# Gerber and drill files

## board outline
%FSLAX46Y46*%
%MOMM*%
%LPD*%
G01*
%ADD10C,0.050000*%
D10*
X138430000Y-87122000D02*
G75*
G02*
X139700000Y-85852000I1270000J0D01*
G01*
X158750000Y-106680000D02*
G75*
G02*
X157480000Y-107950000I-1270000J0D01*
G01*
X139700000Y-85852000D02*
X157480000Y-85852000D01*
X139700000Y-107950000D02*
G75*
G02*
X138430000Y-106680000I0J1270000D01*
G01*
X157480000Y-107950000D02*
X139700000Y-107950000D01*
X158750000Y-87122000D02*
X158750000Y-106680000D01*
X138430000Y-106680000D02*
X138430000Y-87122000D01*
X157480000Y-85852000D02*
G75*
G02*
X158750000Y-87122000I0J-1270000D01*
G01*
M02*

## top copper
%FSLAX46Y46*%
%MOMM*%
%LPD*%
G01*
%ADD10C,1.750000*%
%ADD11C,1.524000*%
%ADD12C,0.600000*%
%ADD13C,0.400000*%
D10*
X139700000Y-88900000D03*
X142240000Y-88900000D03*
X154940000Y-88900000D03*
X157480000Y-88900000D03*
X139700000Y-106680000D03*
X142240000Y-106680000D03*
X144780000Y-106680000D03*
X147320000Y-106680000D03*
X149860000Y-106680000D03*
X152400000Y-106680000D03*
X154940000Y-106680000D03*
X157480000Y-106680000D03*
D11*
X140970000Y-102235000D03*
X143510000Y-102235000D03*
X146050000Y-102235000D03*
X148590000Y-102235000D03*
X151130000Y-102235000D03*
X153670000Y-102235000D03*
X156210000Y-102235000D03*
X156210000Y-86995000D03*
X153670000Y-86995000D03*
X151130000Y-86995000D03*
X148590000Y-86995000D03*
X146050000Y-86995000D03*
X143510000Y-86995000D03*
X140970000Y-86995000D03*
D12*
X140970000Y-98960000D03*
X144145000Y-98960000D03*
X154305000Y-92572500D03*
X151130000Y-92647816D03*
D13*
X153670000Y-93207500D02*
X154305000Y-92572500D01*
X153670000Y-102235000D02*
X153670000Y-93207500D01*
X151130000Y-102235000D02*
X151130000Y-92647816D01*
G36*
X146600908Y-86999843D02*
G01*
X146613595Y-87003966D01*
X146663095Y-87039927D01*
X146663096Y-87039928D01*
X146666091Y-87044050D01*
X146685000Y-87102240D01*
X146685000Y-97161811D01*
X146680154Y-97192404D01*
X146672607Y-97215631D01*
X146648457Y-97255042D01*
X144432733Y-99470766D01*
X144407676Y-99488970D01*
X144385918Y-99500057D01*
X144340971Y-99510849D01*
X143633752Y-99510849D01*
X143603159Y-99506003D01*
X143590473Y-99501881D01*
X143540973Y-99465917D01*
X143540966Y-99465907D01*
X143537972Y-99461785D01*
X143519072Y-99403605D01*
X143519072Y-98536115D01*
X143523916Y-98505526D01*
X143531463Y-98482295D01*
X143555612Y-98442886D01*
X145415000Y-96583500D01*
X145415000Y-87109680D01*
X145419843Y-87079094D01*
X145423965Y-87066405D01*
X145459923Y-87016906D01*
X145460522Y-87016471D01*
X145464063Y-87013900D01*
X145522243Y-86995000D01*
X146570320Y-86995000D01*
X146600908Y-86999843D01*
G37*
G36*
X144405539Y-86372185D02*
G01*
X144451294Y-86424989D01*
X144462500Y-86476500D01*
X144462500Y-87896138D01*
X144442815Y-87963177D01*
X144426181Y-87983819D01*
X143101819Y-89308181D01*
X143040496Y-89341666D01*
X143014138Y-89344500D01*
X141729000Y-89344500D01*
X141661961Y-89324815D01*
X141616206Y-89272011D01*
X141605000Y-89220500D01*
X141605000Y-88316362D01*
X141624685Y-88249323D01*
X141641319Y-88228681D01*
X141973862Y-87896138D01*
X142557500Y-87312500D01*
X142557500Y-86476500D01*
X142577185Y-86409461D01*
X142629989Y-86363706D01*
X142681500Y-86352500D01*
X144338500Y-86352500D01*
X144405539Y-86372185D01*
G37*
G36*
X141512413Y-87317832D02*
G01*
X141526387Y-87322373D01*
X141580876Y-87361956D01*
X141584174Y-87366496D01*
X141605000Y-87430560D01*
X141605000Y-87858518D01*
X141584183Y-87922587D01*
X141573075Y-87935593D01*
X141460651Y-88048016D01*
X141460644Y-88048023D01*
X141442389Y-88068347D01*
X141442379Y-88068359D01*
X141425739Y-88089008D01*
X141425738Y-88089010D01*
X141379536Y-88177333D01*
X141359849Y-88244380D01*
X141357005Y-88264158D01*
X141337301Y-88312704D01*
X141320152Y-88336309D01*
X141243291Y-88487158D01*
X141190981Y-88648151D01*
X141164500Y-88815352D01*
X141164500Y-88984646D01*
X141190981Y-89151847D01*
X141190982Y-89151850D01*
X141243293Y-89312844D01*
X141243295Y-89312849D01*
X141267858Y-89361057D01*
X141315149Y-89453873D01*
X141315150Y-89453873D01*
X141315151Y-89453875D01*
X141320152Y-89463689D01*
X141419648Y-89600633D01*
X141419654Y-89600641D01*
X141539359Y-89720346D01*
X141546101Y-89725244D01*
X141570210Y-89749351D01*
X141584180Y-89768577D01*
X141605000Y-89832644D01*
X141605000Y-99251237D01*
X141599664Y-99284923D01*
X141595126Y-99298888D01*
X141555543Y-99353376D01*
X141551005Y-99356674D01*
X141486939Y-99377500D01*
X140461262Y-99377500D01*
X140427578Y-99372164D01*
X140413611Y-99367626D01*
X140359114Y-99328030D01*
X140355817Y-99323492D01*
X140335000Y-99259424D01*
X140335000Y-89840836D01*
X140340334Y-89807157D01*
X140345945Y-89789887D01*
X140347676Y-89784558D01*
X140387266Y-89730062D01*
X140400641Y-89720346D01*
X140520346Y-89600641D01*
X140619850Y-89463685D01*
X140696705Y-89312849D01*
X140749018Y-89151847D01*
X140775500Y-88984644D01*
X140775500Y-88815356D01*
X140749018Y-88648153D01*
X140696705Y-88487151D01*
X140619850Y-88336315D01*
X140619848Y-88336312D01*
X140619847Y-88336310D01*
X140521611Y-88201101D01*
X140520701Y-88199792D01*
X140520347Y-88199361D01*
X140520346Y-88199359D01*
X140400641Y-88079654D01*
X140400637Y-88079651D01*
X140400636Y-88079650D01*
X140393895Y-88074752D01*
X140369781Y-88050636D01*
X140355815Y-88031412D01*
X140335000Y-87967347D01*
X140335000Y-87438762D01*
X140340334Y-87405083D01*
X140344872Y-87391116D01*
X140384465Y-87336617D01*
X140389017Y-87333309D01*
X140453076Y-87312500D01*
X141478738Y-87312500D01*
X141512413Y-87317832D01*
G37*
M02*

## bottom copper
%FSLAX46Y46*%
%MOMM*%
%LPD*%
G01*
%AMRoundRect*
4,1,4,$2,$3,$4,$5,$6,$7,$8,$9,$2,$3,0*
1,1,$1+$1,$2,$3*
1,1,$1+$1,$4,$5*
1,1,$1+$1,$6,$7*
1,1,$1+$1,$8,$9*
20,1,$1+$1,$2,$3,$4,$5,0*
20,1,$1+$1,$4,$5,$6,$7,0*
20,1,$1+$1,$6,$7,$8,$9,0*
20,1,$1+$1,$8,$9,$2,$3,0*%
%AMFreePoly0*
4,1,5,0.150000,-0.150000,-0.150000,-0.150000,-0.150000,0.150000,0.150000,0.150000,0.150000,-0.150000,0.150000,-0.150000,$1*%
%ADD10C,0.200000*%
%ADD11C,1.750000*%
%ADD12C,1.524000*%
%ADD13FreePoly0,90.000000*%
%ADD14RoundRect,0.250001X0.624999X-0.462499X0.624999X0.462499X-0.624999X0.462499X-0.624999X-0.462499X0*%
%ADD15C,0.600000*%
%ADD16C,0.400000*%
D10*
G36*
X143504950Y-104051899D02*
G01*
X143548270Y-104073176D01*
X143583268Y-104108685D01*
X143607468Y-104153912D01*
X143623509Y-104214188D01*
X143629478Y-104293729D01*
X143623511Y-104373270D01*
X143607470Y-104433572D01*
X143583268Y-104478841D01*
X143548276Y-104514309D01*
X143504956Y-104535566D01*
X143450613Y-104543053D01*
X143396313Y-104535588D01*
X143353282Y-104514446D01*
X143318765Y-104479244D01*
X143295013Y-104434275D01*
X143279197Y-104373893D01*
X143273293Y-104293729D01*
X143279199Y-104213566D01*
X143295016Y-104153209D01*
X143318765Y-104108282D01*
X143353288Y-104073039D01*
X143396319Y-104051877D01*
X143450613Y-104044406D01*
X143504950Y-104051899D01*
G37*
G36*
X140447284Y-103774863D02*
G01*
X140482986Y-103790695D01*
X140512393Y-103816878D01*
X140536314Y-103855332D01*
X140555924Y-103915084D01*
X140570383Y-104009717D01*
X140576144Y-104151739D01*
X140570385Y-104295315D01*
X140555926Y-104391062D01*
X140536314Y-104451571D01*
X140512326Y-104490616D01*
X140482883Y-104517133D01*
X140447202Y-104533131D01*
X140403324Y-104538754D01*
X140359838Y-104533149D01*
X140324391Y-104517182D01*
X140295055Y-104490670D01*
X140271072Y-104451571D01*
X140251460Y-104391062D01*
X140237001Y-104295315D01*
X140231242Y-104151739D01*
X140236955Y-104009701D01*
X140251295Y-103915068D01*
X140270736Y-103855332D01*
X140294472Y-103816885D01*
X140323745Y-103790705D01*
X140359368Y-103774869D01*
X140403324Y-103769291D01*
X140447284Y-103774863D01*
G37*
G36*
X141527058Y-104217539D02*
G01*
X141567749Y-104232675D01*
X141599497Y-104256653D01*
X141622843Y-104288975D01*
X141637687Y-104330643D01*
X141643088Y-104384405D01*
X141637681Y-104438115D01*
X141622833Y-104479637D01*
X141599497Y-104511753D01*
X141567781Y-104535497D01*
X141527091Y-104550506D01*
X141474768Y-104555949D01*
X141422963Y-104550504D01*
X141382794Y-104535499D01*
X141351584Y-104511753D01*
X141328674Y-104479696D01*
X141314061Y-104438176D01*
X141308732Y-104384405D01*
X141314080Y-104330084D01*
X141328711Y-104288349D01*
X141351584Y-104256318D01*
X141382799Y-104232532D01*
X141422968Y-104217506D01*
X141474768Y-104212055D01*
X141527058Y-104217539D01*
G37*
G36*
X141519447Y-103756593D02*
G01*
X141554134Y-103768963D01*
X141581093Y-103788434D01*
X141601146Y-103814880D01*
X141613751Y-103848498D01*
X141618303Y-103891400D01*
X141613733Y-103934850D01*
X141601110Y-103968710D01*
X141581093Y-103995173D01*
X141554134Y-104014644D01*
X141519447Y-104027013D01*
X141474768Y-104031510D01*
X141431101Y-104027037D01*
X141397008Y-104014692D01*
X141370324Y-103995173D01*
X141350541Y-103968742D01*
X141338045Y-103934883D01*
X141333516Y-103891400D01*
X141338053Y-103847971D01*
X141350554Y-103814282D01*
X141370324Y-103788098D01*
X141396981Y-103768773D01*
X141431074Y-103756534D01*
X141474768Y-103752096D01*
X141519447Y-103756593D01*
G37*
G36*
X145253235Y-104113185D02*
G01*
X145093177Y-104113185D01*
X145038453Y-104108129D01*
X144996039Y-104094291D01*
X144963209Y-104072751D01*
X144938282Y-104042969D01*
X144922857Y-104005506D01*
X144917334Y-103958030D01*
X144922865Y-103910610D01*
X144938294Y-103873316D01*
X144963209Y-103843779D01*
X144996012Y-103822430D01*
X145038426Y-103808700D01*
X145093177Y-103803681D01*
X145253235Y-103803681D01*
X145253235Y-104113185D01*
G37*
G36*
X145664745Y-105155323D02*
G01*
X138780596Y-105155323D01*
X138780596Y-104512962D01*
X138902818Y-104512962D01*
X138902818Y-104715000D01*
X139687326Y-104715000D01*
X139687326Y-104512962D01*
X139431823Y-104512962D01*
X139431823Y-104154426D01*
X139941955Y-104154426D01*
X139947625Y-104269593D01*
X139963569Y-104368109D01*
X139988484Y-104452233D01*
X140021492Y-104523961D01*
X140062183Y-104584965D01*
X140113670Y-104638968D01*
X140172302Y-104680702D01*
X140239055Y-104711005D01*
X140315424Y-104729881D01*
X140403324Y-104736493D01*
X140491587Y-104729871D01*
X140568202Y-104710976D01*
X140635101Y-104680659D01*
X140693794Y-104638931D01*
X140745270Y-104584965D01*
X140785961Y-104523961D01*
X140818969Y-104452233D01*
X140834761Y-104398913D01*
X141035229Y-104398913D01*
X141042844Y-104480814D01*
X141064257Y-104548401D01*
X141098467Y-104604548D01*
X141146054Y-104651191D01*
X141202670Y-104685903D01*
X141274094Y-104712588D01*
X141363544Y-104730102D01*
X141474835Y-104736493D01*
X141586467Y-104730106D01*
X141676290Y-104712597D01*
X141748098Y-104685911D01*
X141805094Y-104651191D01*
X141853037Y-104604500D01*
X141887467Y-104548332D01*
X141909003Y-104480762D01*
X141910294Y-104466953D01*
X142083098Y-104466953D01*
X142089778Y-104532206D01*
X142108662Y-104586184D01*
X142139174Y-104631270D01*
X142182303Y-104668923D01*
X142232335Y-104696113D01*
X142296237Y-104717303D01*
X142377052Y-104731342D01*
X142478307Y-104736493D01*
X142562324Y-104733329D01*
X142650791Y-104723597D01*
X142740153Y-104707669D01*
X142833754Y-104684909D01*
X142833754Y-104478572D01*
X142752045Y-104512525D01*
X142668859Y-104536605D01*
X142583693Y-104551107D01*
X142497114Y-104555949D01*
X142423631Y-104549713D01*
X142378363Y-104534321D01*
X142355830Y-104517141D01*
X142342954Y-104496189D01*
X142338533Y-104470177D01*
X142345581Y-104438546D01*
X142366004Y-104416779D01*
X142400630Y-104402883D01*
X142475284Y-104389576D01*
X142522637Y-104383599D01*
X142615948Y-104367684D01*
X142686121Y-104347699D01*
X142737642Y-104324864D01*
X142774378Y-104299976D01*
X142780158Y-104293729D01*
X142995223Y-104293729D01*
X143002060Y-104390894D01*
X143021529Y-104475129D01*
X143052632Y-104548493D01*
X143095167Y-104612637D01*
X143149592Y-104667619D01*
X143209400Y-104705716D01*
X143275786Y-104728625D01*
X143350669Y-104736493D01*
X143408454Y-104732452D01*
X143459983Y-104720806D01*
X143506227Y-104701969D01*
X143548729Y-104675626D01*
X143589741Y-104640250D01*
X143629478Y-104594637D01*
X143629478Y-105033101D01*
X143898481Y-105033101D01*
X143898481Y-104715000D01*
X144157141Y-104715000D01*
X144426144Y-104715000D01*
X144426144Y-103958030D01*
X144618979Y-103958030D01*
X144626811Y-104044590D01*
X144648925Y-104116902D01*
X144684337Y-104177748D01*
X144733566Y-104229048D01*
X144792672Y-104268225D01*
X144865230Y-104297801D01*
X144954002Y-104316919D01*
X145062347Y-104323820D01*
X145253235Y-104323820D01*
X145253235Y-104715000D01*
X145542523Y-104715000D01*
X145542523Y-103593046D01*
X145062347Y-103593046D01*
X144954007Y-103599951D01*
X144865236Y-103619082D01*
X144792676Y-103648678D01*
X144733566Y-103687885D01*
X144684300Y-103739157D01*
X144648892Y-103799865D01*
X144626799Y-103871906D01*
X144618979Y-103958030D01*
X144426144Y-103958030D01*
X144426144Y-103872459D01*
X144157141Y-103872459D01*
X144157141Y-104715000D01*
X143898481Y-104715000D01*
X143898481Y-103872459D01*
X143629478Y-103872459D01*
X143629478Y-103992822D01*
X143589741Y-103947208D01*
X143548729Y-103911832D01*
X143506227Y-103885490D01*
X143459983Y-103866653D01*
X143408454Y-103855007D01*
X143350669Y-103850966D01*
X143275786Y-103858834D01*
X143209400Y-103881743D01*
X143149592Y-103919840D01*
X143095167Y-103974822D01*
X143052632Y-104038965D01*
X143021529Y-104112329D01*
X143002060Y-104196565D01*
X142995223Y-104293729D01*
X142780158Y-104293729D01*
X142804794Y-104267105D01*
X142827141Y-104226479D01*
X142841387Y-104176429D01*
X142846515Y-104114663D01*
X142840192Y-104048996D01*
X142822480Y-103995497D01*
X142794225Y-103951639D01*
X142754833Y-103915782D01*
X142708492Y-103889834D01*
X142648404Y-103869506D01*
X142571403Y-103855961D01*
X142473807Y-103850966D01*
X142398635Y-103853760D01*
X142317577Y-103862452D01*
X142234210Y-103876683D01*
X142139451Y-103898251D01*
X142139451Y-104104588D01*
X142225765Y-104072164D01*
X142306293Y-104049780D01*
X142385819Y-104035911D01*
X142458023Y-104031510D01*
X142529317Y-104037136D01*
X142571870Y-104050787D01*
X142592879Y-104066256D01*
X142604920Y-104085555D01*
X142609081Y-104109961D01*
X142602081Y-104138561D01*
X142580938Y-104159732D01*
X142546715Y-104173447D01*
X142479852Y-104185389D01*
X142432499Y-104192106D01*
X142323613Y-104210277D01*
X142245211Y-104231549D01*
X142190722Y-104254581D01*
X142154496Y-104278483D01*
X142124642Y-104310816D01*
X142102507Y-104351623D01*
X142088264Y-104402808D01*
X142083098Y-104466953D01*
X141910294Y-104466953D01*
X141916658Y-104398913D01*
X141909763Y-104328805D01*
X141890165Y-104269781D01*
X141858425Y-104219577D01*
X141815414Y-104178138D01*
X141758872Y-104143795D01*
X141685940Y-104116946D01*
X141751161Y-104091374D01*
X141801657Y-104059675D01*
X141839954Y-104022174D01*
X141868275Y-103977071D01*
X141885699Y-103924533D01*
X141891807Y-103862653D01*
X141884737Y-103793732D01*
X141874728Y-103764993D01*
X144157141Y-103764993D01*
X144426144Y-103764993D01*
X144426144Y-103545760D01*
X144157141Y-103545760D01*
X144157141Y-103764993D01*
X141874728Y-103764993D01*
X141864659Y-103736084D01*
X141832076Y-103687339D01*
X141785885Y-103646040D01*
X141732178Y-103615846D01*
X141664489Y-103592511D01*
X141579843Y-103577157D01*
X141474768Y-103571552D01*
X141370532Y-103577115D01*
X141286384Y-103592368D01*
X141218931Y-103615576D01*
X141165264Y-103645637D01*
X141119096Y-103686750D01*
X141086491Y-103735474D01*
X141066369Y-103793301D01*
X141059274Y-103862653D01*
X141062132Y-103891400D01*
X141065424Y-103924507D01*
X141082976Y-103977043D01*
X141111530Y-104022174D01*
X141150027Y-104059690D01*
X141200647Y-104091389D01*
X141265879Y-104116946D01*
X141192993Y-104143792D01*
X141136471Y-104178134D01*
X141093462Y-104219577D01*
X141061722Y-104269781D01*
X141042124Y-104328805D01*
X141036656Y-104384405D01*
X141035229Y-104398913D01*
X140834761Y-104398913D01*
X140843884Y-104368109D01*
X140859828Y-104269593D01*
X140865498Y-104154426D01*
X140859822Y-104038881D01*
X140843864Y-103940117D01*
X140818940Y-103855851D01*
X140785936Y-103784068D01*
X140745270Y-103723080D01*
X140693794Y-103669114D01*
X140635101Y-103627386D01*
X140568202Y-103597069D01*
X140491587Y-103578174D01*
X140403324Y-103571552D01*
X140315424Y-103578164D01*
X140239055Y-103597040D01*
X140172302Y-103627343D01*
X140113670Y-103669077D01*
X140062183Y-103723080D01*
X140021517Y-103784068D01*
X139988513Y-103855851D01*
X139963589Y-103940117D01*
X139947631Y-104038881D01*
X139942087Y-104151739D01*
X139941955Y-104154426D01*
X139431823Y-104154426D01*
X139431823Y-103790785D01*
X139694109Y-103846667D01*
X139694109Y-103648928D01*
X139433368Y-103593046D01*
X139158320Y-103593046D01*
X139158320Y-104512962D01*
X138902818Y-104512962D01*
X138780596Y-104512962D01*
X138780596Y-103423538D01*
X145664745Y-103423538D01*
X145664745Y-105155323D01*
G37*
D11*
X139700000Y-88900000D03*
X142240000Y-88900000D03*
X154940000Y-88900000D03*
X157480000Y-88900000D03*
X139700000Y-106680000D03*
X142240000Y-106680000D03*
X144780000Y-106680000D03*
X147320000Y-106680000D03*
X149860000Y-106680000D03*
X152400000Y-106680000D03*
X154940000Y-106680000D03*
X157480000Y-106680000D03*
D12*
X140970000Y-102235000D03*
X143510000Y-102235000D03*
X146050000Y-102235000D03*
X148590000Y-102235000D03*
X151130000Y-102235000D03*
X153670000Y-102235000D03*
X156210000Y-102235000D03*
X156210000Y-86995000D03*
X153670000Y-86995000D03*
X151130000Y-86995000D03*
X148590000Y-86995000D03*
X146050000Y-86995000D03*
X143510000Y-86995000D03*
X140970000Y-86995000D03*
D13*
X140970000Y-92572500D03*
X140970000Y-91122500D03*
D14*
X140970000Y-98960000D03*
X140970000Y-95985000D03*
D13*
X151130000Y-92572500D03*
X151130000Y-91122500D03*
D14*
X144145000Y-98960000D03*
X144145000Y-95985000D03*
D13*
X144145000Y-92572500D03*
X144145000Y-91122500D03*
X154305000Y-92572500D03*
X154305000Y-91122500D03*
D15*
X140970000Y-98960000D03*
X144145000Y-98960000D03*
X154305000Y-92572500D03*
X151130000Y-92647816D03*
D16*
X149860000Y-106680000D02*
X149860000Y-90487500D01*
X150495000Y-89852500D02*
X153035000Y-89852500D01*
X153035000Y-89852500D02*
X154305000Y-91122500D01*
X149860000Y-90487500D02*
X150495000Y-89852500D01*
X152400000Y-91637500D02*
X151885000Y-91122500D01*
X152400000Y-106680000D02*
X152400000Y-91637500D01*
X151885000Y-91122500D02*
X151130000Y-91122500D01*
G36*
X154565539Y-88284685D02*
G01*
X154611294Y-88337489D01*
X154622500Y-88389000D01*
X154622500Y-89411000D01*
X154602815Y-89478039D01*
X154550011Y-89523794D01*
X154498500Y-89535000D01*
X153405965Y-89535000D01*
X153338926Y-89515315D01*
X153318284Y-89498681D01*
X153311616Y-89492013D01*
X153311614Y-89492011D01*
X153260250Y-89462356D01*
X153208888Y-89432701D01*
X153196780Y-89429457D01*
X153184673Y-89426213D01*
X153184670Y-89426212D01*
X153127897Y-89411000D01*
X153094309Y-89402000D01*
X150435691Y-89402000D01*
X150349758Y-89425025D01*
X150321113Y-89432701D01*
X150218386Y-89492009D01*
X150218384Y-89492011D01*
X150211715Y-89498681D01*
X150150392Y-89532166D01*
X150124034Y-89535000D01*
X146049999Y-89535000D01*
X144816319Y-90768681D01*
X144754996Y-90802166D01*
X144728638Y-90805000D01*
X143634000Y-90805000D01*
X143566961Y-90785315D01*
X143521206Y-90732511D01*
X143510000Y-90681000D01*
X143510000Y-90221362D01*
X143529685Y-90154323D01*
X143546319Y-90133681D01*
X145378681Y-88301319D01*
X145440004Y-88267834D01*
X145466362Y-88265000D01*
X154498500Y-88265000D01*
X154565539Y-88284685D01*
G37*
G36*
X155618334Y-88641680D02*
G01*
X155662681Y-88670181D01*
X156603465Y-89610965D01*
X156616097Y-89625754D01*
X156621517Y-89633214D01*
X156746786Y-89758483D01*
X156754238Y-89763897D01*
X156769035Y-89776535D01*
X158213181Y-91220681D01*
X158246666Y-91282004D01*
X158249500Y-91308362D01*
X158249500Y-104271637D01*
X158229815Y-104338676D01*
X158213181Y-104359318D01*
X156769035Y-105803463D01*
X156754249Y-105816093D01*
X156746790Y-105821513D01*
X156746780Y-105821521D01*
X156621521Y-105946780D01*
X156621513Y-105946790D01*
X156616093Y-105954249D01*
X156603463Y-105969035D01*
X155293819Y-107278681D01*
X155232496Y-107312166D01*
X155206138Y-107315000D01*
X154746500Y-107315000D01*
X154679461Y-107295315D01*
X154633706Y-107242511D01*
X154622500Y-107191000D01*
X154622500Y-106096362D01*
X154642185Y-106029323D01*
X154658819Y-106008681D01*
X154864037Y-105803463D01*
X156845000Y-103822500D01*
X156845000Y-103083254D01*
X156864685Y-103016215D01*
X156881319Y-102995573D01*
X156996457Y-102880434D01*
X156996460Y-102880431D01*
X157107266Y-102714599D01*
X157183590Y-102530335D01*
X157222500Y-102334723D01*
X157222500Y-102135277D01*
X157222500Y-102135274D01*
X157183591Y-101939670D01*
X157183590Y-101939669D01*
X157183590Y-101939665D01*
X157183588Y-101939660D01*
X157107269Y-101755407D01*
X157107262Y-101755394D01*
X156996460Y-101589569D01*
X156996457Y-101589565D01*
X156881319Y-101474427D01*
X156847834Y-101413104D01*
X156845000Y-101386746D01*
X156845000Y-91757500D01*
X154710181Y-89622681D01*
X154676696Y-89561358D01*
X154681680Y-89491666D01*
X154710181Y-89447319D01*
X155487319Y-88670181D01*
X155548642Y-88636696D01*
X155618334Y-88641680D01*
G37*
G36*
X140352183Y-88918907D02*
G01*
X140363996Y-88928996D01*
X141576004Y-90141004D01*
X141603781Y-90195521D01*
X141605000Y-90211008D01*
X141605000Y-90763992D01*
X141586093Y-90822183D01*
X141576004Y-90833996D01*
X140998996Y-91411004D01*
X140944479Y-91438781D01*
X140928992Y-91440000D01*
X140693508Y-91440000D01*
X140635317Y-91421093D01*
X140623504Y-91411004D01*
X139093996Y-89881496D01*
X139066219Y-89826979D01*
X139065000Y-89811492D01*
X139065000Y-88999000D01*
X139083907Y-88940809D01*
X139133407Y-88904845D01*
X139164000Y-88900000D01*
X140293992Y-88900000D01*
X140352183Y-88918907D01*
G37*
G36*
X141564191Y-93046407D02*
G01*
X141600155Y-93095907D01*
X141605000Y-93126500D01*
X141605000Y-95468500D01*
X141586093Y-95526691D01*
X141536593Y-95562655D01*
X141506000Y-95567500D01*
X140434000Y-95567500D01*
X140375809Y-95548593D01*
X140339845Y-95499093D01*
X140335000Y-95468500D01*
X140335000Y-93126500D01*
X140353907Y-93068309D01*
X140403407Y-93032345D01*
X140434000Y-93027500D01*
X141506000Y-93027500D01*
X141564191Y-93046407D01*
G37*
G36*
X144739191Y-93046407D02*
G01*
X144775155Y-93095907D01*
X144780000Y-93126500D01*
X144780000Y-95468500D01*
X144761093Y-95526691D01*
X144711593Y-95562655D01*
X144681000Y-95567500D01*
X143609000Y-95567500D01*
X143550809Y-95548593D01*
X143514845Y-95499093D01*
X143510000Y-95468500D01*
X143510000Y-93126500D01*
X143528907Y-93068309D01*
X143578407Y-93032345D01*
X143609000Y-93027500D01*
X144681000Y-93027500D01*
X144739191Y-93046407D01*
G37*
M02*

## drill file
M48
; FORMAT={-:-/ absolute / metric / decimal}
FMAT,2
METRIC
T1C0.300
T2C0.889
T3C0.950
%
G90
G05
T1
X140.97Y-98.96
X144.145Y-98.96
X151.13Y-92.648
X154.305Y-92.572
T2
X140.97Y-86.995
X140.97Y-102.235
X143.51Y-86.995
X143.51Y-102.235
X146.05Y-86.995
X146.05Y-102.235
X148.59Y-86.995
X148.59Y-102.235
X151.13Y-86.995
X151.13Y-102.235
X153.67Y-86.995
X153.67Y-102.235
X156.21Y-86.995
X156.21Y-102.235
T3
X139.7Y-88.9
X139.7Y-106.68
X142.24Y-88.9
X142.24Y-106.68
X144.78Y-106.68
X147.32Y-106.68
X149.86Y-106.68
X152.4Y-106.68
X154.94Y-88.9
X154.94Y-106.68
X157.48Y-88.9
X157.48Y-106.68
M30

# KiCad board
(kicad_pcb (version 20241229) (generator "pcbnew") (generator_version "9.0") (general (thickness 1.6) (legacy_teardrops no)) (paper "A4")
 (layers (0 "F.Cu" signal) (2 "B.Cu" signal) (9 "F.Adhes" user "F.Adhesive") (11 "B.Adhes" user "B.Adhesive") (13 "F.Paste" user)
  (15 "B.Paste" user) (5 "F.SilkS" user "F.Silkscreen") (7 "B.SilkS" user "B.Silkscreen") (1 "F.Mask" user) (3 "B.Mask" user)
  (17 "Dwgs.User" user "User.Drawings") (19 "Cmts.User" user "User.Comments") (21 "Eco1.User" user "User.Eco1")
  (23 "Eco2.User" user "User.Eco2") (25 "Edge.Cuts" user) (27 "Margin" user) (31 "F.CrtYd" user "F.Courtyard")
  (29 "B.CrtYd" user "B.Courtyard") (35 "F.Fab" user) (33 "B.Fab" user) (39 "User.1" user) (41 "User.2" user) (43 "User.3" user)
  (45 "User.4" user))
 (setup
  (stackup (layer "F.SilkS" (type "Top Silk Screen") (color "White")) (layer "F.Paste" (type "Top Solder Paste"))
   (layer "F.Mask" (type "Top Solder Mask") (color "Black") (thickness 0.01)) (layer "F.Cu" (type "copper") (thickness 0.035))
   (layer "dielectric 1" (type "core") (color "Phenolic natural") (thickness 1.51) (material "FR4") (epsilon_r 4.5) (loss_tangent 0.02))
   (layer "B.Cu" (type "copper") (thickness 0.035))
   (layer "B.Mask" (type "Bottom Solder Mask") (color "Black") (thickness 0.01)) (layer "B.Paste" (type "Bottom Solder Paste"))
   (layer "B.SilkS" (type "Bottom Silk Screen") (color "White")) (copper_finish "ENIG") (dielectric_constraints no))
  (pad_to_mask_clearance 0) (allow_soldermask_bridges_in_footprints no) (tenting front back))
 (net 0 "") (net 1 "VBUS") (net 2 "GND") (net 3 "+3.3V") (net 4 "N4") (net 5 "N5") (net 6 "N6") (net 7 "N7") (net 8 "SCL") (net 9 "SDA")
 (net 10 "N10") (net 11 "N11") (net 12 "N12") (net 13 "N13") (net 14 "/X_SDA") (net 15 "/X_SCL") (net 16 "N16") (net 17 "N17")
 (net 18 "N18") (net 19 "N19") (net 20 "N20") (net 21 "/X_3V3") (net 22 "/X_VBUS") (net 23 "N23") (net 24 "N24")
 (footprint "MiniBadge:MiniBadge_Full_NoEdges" (layer "F.Cu") (at 138.43 87.63)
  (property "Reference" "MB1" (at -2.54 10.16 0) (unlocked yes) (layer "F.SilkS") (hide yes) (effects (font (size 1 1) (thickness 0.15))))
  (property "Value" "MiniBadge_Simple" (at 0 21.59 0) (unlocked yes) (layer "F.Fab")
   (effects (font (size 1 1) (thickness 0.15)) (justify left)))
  (pad "1" thru_hole circle (at 1.27 1.27) (size 1.75 1.75) (drill 0.95) (layers "*.Cu" "*.Mask") (remove_unused_layers no) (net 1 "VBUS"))
  (pad "2" thru_hole circle (at 3.81 1.27) (size 1.75 1.75) (drill 0.95) (layers "*.Cu" "*.Mask") (remove_unused_layers no) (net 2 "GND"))
  (pad "7" thru_hole circle (at 16.51 1.27) (size 1.75 1.75) (drill 0.95) (layers "*.Cu" "*.Mask") (remove_unused_layers no) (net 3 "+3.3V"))
  (pad "8" thru_hole circle (at 19.05 1.27) (size 1.75 1.75) (drill 0.95) (layers "*.Cu" "*.Mask") (remove_unused_layers no) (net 2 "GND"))
  (pad "9" thru_hole circle (at 1.27 19.05) (size 1.75 1.75) (drill 0.95) (layers "*.Cu" "*.Mask") (remove_unused_layers no) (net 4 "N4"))
  (pad "10" thru_hole circle (at 3.81 19.05) (size 1.75 1.75) (drill 0.95) (layers "*.Cu" "*.Mask") (remove_unused_layers no) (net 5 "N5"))
  (pad "11" thru_hole circle (at 6.35 19.05) (size 1.75 1.75) (drill 0.95) (layers "*.Cu" "*.Mask") (remove_unused_layers no) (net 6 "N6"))
  (pad "12" thru_hole circle (at 8.89 19.05) (size 1.75 1.75) (drill 0.95) (layers "*.Cu" "*.Mask") (remove_unused_layers no) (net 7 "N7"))
  (pad "13" thru_hole circle (at 11.43 19.05) (size 1.75 1.75) (drill 0.95) (layers "*.Cu" "*.Mask") (remove_unused_layers no) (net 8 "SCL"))
  (pad "14" thru_hole circle (at 13.97 19.05) (size 1.75 1.75) (drill 0.95) (layers "*.Cu" "*.Mask") (remove_unused_layers no) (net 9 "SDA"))
  (pad "15" thru_hole circle (at 16.51 19.05) (size 1.75 1.75) (drill 0.95) (layers "*.Cu" "*.Mask") (remove_unused_layers no)
   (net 3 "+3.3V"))
  (pad "16" thru_hole circle (at 19.05 19.05) (size 1.75 1.75) (drill 0.95) (layers "*.Cu" "*.Mask") (remove_unused_layers no) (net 2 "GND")))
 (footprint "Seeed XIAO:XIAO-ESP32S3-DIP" (layer "F.Cu") (at 148.59 94.615 90)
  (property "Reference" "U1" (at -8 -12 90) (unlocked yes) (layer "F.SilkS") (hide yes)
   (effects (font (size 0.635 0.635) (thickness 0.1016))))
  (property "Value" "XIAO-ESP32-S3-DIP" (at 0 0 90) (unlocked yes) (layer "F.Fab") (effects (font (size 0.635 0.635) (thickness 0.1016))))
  (pad "1" thru_hole circle (at -7.62 -7.62 270) (size 1.524 1.524) (drill 0.889) (layers "*.Cu" "*.Mask") (remove_unused_layers no)
   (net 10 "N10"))
  (pad "2" thru_hole circle (at -7.62 -5.08 270) (size 1.524 1.524) (drill 0.889) (layers "*.Cu" "*.Mask") (remove_unused_layers no)
   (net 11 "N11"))
  (pad "3" thru_hole circle (at -7.62 -2.54 270) (size 1.524 1.524) (drill 0.889) (layers "*.Cu" "*.Mask") (remove_unused_layers no)
   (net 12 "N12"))
  (pad "4" thru_hole circle (at -7.62 0 270) (size 1.524 1.524) (drill 0.889) (layers "*.Cu" "*.Mask") (remove_unused_layers no)
   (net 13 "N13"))
  (pad "5" thru_hole circle (at -7.62 2.54 270) (size 1.524 1.524) (drill 0.889) (layers "*.Cu" "*.Mask") (remove_unused_layers no)
   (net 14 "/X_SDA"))
  (pad "6" thru_hole circle (at -7.62 5.08 270) (size 1.524 1.524) (drill 0.889) (layers "*.Cu" "*.Mask") (remove_unused_layers no)
   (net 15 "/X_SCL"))
  (pad "7" thru_hole circle (at -7.62 7.62 270) (size 1.524 1.524) (drill 0.889) (layers "*.Cu" "*.Mask") (remove_unused_layers no)
   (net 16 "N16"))
  (pad "8" thru_hole circle (at 7.62 7.62 90) (size 1.524 1.524) (drill 0.889) (layers "*.Cu" "*.Mask") (remove_unused_layers no)
   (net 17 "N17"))
  (pad "9" thru_hole circle (at 7.62 5.08 90) (size 1.524 1.524) (drill 0.889) (layers "*.Cu" "*.Mask") (remove_unused_layers no)
   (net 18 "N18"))
  (pad "10" thru_hole circle (at 7.62 2.54 90) (size 1.524 1.524) (drill 0.889) (layers "*.Cu" "*.Mask") (remove_unused_layers no)
   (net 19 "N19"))
  (pad "11" thru_hole circle (at 7.62 0 90) (size 1.524 1.524) (drill 0.889) (layers "*.Cu" "*.Mask") (remove_unused_layers no)
   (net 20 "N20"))
  (pad "12" thru_hole circle (at 7.62 -2.54 90) (size 1.524 1.524) (drill 0.889) (layers "*.Cu" "*.Mask") (remove_unused_layers no)
   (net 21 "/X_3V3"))
  (pad "13" thru_hole circle (at 7.62 -5.08 90) (size 1.524 1.524) (drill 0.889) (layers "*.Cu" "*.Mask") (remove_unused_layers no)
   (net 2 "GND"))
  (pad "14" thru_hole circle (at 7.62 -7.62 90) (size 1.524 1.524) (drill 0.889) (layers "*.Cu" "*.Mask") (remove_unused_layers no)
   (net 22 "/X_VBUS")))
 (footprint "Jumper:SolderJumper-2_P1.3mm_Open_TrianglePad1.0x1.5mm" (layer "B.Cu") (at 140.97 91.8475 90)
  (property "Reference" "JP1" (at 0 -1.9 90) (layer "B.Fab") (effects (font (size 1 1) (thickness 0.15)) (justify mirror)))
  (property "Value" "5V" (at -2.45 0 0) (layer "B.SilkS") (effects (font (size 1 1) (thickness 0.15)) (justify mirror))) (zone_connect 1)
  (pad "1" smd custom (at -0.725 0 90) (size 0.3 0.3) (layers "B.Cu" "B.Mask") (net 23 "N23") (zone_connect 2) (thermal_bridge_angle 45)
   (options (clearance outline) (anchor rect)) (primitives))
  (pad "2" smd custom (at 0.725 0 90) (size 0.3 0.3) (layers "B.Cu" "B.Mask") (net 1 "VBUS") (zone_connect 2) (thermal_bridge_angle 45)
   (options (clearance outline) (anchor rect)) (primitives)))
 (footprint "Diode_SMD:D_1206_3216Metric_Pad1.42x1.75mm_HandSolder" (layer "B.Cu") (at 140.97 97.4725 90)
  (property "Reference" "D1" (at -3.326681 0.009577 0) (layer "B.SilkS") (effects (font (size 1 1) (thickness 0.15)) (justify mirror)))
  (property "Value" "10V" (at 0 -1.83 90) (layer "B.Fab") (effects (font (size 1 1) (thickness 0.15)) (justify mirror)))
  (pad "1" smd roundrect (at -1.4875 0 90) (size 1.425 1.75) (layers "B.Cu" "B.Mask" "B.Paste") (roundrect_rratio 0.175439)
   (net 22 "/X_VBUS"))
  (pad "2" smd roundrect (at 1.4875 0 90) (size 1.425 1.75) (layers "B.Cu" "B.Mask" "B.Paste") (roundrect_rratio 0.175439) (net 23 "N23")))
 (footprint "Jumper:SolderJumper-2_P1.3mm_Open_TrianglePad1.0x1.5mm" (layer "B.Cu") (at 151.13 91.8475 90)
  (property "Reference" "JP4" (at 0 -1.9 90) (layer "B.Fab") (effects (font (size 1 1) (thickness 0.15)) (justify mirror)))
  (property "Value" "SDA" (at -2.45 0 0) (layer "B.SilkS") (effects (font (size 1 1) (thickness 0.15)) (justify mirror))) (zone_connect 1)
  (pad "1" smd custom (at -0.725 0 90) (size 0.3 0.3) (layers "B.Cu" "B.Mask") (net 14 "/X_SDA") (zone_connect 2) (thermal_bridge_angle 45)
   (options (clearance outline) (anchor rect)) (primitives))
  (pad "2" smd custom (at 0.725 0 90) (size 0.3 0.3) (layers "B.Cu" "B.Mask") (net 9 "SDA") (zone_connect 2) (thermal_bridge_angle 45)
   (options (clearance outline) (anchor rect)) (primitives)))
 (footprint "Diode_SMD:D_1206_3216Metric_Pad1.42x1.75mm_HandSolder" (layer "B.Cu") (at 144.145 97.4725 90)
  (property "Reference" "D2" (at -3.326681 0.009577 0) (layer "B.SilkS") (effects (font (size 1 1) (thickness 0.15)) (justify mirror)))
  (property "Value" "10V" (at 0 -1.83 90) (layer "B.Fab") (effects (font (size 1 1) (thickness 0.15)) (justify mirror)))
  (pad "1" smd roundrect (at -1.4875 0 90) (size 1.425 1.75) (layers "B.Cu" "B.Mask" "B.Paste") (roundrect_rratio 0.175439)
   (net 21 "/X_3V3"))
  (pad "2" smd roundrect (at 1.4875 0 90) (size 1.425 1.75) (layers "B.Cu" "B.Mask" "B.Paste") (roundrect_rratio 0.175439) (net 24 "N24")))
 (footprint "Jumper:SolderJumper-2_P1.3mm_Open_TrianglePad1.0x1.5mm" (layer "B.Cu") (at 144.145 91.8475 90)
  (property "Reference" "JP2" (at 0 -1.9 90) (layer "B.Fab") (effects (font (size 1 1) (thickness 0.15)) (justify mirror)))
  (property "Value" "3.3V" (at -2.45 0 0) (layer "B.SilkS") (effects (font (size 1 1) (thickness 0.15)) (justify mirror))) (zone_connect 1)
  (pad "1" smd custom (at -0.725 0 90) (size 0.3 0.3) (layers "B.Cu" "B.Mask") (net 24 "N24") (zone_connect 2) (thermal_bridge_angle 45)
   (options (clearance outline) (anchor rect)) (primitives))
  (pad "2" smd custom (at 0.725 0 90) (size 0.3 0.3) (layers "B.Cu" "B.Mask") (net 3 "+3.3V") (zone_connect 2) (thermal_bridge_angle 45)
   (options (clearance outline) (anchor rect)) (primitives)))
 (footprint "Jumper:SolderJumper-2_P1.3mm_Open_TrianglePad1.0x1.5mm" (layer "B.Cu") (at 154.305 91.8475 90)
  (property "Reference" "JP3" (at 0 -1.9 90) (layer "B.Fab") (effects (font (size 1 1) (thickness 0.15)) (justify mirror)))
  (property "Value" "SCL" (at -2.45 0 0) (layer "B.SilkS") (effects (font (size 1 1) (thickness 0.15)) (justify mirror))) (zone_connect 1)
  (pad "1" smd custom (at -0.725 0 90) (size 0.3 0.3) (layers "B.Cu" "B.Mask") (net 15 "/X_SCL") (zone_connect 2) (thermal_bridge_angle 45)
   (options (clearance outline) (anchor rect)) (primitives))
  (pad "2" smd custom (at 0.725 0 90) (size 0.3 0.3) (layers "B.Cu" "B.Mask") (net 8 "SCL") (zone_connect 2) (thermal_bridge_angle 45)
   (options (clearance outline) (anchor rect)) (primitives)))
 (gr_arc (start 138.43 87.122) (mid 138.801974 86.223974) (end 139.7 85.852) (stroke (width 0.05) (type default)) (layer "Edge.Cuts"))
 (gr_arc (start 158.75 106.68) (mid 158.378026 107.578026) (end 157.48 107.95) (stroke (width 0.05) (type default)) (layer "Edge.Cuts"))
 (gr_line (start 139.7 85.852) (end 157.48 85.852) (stroke (width 0.05) (type default)) (layer "Edge.Cuts"))
 (gr_arc (start 139.7 107.95) (mid 138.801974 107.578026) (end 138.43 106.68) (stroke (width 0.05) (type default)) (layer "Edge.Cuts"))
 (gr_line (start 157.48 107.95) (end 139.7 107.95) (stroke (width 0.05) (type default)) (layer "Edge.Cuts"))
 (gr_line (start 158.75 87.122) (end 158.75 106.68) (stroke (width 0.05) (type default)) (layer "Edge.Cuts"))
 (gr_line (start 138.43 106.68) (end 138.43 87.122) (stroke (width 0.05) (type default)) (layer "Edge.Cuts"))
 (gr_arc (start 157.48 85.852) (mid 158.378026 86.223974) (end 158.75 87.122) (stroke (width 0.05) (type default)) (layer "Edge.Cuts"))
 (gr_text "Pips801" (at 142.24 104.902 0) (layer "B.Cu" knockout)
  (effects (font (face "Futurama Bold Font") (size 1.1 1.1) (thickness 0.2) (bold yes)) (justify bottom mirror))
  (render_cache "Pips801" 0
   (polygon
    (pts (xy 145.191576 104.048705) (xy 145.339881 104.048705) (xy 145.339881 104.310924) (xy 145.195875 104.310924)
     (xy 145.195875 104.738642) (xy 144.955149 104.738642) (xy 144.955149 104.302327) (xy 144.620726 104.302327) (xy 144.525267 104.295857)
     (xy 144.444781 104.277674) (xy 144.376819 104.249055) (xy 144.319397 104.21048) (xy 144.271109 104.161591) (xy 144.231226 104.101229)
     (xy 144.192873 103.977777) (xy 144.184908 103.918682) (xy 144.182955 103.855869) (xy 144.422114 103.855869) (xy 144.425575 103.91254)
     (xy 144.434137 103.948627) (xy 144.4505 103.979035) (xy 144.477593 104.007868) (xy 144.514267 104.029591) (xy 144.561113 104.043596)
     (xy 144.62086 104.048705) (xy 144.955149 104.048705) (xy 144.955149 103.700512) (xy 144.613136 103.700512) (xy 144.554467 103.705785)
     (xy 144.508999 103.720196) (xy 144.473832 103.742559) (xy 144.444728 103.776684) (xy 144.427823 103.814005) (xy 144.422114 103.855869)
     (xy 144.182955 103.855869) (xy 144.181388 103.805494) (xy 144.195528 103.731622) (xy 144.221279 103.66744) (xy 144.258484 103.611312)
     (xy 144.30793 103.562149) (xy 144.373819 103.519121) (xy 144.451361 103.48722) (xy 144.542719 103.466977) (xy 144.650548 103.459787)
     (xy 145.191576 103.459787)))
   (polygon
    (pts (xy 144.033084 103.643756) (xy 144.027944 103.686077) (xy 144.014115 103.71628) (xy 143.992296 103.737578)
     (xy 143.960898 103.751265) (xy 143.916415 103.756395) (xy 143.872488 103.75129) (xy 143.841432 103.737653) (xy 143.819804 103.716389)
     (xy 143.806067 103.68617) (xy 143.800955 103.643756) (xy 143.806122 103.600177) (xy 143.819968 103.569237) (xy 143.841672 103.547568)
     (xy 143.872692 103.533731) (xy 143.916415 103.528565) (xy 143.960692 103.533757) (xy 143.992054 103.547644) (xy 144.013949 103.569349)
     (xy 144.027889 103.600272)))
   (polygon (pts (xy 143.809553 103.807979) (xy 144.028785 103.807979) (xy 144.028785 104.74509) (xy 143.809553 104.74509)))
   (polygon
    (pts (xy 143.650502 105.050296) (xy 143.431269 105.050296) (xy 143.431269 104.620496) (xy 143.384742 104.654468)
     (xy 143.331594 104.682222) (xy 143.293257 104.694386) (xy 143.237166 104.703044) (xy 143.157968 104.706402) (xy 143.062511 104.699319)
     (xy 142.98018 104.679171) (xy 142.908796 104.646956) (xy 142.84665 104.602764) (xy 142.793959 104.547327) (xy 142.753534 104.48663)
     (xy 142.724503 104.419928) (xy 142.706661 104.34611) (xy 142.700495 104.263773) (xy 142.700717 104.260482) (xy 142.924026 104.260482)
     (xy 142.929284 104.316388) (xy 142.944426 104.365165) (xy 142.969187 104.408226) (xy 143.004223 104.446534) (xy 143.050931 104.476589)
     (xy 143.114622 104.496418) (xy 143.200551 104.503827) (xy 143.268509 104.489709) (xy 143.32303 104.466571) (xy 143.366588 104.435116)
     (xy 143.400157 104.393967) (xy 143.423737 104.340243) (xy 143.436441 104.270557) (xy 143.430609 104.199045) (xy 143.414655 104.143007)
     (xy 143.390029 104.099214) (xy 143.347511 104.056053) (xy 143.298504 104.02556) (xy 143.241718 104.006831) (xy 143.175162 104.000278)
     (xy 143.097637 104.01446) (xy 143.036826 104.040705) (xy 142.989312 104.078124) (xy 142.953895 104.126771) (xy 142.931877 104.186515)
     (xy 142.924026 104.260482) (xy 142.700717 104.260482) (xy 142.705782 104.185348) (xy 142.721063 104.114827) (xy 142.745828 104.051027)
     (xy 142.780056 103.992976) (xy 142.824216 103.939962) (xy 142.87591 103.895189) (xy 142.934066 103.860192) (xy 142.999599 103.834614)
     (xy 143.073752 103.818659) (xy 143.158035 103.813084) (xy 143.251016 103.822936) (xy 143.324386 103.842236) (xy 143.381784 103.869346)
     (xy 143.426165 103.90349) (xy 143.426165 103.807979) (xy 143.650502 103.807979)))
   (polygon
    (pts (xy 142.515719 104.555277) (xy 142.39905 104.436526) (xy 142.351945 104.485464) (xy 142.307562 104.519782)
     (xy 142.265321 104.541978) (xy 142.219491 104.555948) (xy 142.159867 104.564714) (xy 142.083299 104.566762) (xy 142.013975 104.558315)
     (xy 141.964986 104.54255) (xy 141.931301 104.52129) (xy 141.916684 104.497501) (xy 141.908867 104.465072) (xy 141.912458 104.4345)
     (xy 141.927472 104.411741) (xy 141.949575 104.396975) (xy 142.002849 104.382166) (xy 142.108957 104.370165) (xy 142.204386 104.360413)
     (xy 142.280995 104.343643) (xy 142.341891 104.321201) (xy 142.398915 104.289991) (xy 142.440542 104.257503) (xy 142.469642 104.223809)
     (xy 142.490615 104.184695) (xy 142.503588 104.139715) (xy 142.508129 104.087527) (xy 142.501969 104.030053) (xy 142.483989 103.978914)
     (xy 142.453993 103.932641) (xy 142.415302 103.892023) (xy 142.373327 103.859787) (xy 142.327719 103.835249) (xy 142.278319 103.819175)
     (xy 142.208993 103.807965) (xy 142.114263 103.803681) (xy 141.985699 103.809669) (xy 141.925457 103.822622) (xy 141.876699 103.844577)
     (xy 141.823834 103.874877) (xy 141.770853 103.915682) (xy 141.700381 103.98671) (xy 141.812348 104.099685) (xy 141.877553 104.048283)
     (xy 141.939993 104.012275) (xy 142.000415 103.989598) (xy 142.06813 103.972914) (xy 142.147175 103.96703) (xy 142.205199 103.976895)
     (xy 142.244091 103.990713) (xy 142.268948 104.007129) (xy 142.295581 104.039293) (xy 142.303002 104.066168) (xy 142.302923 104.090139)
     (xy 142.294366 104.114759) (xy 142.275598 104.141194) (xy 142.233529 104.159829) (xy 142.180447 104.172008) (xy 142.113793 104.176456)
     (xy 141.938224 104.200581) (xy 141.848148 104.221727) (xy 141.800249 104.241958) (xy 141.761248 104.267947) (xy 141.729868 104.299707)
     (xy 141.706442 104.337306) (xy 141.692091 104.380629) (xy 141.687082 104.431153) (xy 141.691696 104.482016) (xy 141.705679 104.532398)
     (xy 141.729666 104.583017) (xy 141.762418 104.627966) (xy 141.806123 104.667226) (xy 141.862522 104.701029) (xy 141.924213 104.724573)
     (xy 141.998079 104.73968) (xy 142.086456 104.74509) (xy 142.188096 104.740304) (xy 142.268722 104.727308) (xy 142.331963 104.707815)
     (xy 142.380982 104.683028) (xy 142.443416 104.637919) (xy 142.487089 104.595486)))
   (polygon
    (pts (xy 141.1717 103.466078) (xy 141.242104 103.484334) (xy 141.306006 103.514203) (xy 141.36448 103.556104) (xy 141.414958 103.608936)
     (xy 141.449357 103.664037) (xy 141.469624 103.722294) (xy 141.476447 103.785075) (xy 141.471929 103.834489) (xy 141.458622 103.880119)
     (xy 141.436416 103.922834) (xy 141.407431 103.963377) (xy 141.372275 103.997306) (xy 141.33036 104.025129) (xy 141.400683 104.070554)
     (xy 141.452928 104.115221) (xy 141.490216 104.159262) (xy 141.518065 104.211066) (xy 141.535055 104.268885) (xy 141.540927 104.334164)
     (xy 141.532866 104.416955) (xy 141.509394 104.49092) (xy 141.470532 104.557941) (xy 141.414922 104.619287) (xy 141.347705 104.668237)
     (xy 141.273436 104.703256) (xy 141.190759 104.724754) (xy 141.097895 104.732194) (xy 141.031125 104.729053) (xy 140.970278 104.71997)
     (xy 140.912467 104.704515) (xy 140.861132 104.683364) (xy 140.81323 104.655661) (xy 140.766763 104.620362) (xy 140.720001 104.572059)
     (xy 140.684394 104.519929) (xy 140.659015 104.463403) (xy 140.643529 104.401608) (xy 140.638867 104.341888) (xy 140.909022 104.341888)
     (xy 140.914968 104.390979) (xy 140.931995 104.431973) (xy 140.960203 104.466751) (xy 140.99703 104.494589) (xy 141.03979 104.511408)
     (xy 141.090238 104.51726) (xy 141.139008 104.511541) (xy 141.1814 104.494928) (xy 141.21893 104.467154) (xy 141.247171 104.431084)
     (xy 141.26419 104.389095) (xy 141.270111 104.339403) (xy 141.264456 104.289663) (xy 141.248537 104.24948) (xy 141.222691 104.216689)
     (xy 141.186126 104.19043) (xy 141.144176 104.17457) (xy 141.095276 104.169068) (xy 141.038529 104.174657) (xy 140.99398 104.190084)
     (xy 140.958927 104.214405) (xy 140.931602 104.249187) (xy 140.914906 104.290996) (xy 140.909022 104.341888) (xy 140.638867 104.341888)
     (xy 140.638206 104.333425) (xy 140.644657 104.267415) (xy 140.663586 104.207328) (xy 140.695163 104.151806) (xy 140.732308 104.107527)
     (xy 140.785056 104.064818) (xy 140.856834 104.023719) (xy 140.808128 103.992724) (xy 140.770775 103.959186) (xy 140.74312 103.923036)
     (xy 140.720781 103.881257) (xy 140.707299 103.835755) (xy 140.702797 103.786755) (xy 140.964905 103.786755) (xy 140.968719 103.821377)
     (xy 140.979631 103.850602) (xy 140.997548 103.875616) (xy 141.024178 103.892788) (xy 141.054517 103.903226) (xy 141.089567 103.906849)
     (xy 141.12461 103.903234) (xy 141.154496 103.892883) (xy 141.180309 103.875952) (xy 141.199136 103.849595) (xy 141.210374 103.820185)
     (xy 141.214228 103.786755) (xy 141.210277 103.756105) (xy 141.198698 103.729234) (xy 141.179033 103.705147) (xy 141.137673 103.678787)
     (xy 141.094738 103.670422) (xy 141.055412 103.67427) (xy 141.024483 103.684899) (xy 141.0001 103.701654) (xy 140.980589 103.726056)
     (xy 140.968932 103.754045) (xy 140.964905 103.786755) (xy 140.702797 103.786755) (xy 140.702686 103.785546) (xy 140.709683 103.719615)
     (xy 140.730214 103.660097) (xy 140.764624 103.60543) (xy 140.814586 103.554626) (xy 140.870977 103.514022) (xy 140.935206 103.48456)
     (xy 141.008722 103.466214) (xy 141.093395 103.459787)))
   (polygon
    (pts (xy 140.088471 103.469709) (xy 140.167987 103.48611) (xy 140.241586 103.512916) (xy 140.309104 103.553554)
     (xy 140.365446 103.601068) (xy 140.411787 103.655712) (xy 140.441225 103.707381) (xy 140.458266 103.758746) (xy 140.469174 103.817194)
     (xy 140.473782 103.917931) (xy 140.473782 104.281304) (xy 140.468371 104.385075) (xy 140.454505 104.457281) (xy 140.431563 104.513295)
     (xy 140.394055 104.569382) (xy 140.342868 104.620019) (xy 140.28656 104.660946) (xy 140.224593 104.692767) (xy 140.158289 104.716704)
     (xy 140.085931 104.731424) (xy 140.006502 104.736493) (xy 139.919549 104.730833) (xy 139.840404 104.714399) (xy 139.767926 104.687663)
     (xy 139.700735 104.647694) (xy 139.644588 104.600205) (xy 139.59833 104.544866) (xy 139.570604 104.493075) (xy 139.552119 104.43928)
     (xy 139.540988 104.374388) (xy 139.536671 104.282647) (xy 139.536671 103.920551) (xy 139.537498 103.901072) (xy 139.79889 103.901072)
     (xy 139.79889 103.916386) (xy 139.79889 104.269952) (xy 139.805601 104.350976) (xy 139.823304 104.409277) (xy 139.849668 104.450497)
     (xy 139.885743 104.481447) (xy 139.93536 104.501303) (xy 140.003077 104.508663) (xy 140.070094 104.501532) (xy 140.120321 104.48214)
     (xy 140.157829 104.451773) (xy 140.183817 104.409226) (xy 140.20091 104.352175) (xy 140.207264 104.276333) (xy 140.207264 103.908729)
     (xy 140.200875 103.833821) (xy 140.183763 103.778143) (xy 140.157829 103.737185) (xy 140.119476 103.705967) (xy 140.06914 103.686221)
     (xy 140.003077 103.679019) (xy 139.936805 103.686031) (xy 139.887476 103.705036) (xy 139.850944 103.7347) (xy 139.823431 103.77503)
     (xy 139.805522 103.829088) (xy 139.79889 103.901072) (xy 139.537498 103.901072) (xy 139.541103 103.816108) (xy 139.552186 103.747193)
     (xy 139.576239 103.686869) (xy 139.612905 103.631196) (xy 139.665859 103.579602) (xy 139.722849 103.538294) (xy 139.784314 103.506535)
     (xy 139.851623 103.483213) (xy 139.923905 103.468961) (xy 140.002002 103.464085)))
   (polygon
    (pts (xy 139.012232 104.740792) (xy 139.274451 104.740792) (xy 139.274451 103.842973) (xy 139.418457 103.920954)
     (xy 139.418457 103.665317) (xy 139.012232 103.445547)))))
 (segment (start 149.86 106.68) (end 149.86 90.4875) (width 0.4) (layer "B.Cu") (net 8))
 (segment (start 150.495 89.8525) (end 153.035 89.8525) (width 0.4) (layer "B.Cu") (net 8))
 (segment (start 153.035 89.8525) (end 154.305 91.1225) (width 0.4) (layer "B.Cu") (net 8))
 (segment (start 149.86 90.4875) (end 150.495 89.8525) (width 0.4) (layer "B.Cu") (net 8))
 (segment (start 152.4 91.6375) (end 151.885 91.1225) (width 0.4) (layer "B.Cu") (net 9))
 (segment (start 152.4 106.68) (end 152.4 91.6375) (width 0.4) (layer "B.Cu") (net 9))
 (segment (start 151.885 91.1225) (end 151.13 91.1225) (width 0.4) (layer "B.Cu") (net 9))
 (via (at 140.97 98.96) (size 0.6) (drill 0.3) (layers "F.Cu" "B.Cu") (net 22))
 (via (at 144.145 98.96) (size 0.6) (drill 0.3) (layers "F.Cu" "B.Cu") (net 21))
 (segment (start 153.67 93.2075) (end 154.305 92.5725) (width 0.4) (layer "F.Cu") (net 15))
 (segment (start 153.67 102.235) (end 153.67 93.2075) (width 0.4) (layer "F.Cu") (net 15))
 (via (at 154.305 92.5725) (size 0.6) (drill 0.3) (layers "F.Cu" "B.Cu") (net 15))
 (segment (start 151.13 102.235) (end 151.13 92.647816) (width 0.4) (layer "F.Cu") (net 14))
 (via (at 151.13 92.647816) (size 0.6) (drill 0.3) (layers "F.Cu" "B.Cu") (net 14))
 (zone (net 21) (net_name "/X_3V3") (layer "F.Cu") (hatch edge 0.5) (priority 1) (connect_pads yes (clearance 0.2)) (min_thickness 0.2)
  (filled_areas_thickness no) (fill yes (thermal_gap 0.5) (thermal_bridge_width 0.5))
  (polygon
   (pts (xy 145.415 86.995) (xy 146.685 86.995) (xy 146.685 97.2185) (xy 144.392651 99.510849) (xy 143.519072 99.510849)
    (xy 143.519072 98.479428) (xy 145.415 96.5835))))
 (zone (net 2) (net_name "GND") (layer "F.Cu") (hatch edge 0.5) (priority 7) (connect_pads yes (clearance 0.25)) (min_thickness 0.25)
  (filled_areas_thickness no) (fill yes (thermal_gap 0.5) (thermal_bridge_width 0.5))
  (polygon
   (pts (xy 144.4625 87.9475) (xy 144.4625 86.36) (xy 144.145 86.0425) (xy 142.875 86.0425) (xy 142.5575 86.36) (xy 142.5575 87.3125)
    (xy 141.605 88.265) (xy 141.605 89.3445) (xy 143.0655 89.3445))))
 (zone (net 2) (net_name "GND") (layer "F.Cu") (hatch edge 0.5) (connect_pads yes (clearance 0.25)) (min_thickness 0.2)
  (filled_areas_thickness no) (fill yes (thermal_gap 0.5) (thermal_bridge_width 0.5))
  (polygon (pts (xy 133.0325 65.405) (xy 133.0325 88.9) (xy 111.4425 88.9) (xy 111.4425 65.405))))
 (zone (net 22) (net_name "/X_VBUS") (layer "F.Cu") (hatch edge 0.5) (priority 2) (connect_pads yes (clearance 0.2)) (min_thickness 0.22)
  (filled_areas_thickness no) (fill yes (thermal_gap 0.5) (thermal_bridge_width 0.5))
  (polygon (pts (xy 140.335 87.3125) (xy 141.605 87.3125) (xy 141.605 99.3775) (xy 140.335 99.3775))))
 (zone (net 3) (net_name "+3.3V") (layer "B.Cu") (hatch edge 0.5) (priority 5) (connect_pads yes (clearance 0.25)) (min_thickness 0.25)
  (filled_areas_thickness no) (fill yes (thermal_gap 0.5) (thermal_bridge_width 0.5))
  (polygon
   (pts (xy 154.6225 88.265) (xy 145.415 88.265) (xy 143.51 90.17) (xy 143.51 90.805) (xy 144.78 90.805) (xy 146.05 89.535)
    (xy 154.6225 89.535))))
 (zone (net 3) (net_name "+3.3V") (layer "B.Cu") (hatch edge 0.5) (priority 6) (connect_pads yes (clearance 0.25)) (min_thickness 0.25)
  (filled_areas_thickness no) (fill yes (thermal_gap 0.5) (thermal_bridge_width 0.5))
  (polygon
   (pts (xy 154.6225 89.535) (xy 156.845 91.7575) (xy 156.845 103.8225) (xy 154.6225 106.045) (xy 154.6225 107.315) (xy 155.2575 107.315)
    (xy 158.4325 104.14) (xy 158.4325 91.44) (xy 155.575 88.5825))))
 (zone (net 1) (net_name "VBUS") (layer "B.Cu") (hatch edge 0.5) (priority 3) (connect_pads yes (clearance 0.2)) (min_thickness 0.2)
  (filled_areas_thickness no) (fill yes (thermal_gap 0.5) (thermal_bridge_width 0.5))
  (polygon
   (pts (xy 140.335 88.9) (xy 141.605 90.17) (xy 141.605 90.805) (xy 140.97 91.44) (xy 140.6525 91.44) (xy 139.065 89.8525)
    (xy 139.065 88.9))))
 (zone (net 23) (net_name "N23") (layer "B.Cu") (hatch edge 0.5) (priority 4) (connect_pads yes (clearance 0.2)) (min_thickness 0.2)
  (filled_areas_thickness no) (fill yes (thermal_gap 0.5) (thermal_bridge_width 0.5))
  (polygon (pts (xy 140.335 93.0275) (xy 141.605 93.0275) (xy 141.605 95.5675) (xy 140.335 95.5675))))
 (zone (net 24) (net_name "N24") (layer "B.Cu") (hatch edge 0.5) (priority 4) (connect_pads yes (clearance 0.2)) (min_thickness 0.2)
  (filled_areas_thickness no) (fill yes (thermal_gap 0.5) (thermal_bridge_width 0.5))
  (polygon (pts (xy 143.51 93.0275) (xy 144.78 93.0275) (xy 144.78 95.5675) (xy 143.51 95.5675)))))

